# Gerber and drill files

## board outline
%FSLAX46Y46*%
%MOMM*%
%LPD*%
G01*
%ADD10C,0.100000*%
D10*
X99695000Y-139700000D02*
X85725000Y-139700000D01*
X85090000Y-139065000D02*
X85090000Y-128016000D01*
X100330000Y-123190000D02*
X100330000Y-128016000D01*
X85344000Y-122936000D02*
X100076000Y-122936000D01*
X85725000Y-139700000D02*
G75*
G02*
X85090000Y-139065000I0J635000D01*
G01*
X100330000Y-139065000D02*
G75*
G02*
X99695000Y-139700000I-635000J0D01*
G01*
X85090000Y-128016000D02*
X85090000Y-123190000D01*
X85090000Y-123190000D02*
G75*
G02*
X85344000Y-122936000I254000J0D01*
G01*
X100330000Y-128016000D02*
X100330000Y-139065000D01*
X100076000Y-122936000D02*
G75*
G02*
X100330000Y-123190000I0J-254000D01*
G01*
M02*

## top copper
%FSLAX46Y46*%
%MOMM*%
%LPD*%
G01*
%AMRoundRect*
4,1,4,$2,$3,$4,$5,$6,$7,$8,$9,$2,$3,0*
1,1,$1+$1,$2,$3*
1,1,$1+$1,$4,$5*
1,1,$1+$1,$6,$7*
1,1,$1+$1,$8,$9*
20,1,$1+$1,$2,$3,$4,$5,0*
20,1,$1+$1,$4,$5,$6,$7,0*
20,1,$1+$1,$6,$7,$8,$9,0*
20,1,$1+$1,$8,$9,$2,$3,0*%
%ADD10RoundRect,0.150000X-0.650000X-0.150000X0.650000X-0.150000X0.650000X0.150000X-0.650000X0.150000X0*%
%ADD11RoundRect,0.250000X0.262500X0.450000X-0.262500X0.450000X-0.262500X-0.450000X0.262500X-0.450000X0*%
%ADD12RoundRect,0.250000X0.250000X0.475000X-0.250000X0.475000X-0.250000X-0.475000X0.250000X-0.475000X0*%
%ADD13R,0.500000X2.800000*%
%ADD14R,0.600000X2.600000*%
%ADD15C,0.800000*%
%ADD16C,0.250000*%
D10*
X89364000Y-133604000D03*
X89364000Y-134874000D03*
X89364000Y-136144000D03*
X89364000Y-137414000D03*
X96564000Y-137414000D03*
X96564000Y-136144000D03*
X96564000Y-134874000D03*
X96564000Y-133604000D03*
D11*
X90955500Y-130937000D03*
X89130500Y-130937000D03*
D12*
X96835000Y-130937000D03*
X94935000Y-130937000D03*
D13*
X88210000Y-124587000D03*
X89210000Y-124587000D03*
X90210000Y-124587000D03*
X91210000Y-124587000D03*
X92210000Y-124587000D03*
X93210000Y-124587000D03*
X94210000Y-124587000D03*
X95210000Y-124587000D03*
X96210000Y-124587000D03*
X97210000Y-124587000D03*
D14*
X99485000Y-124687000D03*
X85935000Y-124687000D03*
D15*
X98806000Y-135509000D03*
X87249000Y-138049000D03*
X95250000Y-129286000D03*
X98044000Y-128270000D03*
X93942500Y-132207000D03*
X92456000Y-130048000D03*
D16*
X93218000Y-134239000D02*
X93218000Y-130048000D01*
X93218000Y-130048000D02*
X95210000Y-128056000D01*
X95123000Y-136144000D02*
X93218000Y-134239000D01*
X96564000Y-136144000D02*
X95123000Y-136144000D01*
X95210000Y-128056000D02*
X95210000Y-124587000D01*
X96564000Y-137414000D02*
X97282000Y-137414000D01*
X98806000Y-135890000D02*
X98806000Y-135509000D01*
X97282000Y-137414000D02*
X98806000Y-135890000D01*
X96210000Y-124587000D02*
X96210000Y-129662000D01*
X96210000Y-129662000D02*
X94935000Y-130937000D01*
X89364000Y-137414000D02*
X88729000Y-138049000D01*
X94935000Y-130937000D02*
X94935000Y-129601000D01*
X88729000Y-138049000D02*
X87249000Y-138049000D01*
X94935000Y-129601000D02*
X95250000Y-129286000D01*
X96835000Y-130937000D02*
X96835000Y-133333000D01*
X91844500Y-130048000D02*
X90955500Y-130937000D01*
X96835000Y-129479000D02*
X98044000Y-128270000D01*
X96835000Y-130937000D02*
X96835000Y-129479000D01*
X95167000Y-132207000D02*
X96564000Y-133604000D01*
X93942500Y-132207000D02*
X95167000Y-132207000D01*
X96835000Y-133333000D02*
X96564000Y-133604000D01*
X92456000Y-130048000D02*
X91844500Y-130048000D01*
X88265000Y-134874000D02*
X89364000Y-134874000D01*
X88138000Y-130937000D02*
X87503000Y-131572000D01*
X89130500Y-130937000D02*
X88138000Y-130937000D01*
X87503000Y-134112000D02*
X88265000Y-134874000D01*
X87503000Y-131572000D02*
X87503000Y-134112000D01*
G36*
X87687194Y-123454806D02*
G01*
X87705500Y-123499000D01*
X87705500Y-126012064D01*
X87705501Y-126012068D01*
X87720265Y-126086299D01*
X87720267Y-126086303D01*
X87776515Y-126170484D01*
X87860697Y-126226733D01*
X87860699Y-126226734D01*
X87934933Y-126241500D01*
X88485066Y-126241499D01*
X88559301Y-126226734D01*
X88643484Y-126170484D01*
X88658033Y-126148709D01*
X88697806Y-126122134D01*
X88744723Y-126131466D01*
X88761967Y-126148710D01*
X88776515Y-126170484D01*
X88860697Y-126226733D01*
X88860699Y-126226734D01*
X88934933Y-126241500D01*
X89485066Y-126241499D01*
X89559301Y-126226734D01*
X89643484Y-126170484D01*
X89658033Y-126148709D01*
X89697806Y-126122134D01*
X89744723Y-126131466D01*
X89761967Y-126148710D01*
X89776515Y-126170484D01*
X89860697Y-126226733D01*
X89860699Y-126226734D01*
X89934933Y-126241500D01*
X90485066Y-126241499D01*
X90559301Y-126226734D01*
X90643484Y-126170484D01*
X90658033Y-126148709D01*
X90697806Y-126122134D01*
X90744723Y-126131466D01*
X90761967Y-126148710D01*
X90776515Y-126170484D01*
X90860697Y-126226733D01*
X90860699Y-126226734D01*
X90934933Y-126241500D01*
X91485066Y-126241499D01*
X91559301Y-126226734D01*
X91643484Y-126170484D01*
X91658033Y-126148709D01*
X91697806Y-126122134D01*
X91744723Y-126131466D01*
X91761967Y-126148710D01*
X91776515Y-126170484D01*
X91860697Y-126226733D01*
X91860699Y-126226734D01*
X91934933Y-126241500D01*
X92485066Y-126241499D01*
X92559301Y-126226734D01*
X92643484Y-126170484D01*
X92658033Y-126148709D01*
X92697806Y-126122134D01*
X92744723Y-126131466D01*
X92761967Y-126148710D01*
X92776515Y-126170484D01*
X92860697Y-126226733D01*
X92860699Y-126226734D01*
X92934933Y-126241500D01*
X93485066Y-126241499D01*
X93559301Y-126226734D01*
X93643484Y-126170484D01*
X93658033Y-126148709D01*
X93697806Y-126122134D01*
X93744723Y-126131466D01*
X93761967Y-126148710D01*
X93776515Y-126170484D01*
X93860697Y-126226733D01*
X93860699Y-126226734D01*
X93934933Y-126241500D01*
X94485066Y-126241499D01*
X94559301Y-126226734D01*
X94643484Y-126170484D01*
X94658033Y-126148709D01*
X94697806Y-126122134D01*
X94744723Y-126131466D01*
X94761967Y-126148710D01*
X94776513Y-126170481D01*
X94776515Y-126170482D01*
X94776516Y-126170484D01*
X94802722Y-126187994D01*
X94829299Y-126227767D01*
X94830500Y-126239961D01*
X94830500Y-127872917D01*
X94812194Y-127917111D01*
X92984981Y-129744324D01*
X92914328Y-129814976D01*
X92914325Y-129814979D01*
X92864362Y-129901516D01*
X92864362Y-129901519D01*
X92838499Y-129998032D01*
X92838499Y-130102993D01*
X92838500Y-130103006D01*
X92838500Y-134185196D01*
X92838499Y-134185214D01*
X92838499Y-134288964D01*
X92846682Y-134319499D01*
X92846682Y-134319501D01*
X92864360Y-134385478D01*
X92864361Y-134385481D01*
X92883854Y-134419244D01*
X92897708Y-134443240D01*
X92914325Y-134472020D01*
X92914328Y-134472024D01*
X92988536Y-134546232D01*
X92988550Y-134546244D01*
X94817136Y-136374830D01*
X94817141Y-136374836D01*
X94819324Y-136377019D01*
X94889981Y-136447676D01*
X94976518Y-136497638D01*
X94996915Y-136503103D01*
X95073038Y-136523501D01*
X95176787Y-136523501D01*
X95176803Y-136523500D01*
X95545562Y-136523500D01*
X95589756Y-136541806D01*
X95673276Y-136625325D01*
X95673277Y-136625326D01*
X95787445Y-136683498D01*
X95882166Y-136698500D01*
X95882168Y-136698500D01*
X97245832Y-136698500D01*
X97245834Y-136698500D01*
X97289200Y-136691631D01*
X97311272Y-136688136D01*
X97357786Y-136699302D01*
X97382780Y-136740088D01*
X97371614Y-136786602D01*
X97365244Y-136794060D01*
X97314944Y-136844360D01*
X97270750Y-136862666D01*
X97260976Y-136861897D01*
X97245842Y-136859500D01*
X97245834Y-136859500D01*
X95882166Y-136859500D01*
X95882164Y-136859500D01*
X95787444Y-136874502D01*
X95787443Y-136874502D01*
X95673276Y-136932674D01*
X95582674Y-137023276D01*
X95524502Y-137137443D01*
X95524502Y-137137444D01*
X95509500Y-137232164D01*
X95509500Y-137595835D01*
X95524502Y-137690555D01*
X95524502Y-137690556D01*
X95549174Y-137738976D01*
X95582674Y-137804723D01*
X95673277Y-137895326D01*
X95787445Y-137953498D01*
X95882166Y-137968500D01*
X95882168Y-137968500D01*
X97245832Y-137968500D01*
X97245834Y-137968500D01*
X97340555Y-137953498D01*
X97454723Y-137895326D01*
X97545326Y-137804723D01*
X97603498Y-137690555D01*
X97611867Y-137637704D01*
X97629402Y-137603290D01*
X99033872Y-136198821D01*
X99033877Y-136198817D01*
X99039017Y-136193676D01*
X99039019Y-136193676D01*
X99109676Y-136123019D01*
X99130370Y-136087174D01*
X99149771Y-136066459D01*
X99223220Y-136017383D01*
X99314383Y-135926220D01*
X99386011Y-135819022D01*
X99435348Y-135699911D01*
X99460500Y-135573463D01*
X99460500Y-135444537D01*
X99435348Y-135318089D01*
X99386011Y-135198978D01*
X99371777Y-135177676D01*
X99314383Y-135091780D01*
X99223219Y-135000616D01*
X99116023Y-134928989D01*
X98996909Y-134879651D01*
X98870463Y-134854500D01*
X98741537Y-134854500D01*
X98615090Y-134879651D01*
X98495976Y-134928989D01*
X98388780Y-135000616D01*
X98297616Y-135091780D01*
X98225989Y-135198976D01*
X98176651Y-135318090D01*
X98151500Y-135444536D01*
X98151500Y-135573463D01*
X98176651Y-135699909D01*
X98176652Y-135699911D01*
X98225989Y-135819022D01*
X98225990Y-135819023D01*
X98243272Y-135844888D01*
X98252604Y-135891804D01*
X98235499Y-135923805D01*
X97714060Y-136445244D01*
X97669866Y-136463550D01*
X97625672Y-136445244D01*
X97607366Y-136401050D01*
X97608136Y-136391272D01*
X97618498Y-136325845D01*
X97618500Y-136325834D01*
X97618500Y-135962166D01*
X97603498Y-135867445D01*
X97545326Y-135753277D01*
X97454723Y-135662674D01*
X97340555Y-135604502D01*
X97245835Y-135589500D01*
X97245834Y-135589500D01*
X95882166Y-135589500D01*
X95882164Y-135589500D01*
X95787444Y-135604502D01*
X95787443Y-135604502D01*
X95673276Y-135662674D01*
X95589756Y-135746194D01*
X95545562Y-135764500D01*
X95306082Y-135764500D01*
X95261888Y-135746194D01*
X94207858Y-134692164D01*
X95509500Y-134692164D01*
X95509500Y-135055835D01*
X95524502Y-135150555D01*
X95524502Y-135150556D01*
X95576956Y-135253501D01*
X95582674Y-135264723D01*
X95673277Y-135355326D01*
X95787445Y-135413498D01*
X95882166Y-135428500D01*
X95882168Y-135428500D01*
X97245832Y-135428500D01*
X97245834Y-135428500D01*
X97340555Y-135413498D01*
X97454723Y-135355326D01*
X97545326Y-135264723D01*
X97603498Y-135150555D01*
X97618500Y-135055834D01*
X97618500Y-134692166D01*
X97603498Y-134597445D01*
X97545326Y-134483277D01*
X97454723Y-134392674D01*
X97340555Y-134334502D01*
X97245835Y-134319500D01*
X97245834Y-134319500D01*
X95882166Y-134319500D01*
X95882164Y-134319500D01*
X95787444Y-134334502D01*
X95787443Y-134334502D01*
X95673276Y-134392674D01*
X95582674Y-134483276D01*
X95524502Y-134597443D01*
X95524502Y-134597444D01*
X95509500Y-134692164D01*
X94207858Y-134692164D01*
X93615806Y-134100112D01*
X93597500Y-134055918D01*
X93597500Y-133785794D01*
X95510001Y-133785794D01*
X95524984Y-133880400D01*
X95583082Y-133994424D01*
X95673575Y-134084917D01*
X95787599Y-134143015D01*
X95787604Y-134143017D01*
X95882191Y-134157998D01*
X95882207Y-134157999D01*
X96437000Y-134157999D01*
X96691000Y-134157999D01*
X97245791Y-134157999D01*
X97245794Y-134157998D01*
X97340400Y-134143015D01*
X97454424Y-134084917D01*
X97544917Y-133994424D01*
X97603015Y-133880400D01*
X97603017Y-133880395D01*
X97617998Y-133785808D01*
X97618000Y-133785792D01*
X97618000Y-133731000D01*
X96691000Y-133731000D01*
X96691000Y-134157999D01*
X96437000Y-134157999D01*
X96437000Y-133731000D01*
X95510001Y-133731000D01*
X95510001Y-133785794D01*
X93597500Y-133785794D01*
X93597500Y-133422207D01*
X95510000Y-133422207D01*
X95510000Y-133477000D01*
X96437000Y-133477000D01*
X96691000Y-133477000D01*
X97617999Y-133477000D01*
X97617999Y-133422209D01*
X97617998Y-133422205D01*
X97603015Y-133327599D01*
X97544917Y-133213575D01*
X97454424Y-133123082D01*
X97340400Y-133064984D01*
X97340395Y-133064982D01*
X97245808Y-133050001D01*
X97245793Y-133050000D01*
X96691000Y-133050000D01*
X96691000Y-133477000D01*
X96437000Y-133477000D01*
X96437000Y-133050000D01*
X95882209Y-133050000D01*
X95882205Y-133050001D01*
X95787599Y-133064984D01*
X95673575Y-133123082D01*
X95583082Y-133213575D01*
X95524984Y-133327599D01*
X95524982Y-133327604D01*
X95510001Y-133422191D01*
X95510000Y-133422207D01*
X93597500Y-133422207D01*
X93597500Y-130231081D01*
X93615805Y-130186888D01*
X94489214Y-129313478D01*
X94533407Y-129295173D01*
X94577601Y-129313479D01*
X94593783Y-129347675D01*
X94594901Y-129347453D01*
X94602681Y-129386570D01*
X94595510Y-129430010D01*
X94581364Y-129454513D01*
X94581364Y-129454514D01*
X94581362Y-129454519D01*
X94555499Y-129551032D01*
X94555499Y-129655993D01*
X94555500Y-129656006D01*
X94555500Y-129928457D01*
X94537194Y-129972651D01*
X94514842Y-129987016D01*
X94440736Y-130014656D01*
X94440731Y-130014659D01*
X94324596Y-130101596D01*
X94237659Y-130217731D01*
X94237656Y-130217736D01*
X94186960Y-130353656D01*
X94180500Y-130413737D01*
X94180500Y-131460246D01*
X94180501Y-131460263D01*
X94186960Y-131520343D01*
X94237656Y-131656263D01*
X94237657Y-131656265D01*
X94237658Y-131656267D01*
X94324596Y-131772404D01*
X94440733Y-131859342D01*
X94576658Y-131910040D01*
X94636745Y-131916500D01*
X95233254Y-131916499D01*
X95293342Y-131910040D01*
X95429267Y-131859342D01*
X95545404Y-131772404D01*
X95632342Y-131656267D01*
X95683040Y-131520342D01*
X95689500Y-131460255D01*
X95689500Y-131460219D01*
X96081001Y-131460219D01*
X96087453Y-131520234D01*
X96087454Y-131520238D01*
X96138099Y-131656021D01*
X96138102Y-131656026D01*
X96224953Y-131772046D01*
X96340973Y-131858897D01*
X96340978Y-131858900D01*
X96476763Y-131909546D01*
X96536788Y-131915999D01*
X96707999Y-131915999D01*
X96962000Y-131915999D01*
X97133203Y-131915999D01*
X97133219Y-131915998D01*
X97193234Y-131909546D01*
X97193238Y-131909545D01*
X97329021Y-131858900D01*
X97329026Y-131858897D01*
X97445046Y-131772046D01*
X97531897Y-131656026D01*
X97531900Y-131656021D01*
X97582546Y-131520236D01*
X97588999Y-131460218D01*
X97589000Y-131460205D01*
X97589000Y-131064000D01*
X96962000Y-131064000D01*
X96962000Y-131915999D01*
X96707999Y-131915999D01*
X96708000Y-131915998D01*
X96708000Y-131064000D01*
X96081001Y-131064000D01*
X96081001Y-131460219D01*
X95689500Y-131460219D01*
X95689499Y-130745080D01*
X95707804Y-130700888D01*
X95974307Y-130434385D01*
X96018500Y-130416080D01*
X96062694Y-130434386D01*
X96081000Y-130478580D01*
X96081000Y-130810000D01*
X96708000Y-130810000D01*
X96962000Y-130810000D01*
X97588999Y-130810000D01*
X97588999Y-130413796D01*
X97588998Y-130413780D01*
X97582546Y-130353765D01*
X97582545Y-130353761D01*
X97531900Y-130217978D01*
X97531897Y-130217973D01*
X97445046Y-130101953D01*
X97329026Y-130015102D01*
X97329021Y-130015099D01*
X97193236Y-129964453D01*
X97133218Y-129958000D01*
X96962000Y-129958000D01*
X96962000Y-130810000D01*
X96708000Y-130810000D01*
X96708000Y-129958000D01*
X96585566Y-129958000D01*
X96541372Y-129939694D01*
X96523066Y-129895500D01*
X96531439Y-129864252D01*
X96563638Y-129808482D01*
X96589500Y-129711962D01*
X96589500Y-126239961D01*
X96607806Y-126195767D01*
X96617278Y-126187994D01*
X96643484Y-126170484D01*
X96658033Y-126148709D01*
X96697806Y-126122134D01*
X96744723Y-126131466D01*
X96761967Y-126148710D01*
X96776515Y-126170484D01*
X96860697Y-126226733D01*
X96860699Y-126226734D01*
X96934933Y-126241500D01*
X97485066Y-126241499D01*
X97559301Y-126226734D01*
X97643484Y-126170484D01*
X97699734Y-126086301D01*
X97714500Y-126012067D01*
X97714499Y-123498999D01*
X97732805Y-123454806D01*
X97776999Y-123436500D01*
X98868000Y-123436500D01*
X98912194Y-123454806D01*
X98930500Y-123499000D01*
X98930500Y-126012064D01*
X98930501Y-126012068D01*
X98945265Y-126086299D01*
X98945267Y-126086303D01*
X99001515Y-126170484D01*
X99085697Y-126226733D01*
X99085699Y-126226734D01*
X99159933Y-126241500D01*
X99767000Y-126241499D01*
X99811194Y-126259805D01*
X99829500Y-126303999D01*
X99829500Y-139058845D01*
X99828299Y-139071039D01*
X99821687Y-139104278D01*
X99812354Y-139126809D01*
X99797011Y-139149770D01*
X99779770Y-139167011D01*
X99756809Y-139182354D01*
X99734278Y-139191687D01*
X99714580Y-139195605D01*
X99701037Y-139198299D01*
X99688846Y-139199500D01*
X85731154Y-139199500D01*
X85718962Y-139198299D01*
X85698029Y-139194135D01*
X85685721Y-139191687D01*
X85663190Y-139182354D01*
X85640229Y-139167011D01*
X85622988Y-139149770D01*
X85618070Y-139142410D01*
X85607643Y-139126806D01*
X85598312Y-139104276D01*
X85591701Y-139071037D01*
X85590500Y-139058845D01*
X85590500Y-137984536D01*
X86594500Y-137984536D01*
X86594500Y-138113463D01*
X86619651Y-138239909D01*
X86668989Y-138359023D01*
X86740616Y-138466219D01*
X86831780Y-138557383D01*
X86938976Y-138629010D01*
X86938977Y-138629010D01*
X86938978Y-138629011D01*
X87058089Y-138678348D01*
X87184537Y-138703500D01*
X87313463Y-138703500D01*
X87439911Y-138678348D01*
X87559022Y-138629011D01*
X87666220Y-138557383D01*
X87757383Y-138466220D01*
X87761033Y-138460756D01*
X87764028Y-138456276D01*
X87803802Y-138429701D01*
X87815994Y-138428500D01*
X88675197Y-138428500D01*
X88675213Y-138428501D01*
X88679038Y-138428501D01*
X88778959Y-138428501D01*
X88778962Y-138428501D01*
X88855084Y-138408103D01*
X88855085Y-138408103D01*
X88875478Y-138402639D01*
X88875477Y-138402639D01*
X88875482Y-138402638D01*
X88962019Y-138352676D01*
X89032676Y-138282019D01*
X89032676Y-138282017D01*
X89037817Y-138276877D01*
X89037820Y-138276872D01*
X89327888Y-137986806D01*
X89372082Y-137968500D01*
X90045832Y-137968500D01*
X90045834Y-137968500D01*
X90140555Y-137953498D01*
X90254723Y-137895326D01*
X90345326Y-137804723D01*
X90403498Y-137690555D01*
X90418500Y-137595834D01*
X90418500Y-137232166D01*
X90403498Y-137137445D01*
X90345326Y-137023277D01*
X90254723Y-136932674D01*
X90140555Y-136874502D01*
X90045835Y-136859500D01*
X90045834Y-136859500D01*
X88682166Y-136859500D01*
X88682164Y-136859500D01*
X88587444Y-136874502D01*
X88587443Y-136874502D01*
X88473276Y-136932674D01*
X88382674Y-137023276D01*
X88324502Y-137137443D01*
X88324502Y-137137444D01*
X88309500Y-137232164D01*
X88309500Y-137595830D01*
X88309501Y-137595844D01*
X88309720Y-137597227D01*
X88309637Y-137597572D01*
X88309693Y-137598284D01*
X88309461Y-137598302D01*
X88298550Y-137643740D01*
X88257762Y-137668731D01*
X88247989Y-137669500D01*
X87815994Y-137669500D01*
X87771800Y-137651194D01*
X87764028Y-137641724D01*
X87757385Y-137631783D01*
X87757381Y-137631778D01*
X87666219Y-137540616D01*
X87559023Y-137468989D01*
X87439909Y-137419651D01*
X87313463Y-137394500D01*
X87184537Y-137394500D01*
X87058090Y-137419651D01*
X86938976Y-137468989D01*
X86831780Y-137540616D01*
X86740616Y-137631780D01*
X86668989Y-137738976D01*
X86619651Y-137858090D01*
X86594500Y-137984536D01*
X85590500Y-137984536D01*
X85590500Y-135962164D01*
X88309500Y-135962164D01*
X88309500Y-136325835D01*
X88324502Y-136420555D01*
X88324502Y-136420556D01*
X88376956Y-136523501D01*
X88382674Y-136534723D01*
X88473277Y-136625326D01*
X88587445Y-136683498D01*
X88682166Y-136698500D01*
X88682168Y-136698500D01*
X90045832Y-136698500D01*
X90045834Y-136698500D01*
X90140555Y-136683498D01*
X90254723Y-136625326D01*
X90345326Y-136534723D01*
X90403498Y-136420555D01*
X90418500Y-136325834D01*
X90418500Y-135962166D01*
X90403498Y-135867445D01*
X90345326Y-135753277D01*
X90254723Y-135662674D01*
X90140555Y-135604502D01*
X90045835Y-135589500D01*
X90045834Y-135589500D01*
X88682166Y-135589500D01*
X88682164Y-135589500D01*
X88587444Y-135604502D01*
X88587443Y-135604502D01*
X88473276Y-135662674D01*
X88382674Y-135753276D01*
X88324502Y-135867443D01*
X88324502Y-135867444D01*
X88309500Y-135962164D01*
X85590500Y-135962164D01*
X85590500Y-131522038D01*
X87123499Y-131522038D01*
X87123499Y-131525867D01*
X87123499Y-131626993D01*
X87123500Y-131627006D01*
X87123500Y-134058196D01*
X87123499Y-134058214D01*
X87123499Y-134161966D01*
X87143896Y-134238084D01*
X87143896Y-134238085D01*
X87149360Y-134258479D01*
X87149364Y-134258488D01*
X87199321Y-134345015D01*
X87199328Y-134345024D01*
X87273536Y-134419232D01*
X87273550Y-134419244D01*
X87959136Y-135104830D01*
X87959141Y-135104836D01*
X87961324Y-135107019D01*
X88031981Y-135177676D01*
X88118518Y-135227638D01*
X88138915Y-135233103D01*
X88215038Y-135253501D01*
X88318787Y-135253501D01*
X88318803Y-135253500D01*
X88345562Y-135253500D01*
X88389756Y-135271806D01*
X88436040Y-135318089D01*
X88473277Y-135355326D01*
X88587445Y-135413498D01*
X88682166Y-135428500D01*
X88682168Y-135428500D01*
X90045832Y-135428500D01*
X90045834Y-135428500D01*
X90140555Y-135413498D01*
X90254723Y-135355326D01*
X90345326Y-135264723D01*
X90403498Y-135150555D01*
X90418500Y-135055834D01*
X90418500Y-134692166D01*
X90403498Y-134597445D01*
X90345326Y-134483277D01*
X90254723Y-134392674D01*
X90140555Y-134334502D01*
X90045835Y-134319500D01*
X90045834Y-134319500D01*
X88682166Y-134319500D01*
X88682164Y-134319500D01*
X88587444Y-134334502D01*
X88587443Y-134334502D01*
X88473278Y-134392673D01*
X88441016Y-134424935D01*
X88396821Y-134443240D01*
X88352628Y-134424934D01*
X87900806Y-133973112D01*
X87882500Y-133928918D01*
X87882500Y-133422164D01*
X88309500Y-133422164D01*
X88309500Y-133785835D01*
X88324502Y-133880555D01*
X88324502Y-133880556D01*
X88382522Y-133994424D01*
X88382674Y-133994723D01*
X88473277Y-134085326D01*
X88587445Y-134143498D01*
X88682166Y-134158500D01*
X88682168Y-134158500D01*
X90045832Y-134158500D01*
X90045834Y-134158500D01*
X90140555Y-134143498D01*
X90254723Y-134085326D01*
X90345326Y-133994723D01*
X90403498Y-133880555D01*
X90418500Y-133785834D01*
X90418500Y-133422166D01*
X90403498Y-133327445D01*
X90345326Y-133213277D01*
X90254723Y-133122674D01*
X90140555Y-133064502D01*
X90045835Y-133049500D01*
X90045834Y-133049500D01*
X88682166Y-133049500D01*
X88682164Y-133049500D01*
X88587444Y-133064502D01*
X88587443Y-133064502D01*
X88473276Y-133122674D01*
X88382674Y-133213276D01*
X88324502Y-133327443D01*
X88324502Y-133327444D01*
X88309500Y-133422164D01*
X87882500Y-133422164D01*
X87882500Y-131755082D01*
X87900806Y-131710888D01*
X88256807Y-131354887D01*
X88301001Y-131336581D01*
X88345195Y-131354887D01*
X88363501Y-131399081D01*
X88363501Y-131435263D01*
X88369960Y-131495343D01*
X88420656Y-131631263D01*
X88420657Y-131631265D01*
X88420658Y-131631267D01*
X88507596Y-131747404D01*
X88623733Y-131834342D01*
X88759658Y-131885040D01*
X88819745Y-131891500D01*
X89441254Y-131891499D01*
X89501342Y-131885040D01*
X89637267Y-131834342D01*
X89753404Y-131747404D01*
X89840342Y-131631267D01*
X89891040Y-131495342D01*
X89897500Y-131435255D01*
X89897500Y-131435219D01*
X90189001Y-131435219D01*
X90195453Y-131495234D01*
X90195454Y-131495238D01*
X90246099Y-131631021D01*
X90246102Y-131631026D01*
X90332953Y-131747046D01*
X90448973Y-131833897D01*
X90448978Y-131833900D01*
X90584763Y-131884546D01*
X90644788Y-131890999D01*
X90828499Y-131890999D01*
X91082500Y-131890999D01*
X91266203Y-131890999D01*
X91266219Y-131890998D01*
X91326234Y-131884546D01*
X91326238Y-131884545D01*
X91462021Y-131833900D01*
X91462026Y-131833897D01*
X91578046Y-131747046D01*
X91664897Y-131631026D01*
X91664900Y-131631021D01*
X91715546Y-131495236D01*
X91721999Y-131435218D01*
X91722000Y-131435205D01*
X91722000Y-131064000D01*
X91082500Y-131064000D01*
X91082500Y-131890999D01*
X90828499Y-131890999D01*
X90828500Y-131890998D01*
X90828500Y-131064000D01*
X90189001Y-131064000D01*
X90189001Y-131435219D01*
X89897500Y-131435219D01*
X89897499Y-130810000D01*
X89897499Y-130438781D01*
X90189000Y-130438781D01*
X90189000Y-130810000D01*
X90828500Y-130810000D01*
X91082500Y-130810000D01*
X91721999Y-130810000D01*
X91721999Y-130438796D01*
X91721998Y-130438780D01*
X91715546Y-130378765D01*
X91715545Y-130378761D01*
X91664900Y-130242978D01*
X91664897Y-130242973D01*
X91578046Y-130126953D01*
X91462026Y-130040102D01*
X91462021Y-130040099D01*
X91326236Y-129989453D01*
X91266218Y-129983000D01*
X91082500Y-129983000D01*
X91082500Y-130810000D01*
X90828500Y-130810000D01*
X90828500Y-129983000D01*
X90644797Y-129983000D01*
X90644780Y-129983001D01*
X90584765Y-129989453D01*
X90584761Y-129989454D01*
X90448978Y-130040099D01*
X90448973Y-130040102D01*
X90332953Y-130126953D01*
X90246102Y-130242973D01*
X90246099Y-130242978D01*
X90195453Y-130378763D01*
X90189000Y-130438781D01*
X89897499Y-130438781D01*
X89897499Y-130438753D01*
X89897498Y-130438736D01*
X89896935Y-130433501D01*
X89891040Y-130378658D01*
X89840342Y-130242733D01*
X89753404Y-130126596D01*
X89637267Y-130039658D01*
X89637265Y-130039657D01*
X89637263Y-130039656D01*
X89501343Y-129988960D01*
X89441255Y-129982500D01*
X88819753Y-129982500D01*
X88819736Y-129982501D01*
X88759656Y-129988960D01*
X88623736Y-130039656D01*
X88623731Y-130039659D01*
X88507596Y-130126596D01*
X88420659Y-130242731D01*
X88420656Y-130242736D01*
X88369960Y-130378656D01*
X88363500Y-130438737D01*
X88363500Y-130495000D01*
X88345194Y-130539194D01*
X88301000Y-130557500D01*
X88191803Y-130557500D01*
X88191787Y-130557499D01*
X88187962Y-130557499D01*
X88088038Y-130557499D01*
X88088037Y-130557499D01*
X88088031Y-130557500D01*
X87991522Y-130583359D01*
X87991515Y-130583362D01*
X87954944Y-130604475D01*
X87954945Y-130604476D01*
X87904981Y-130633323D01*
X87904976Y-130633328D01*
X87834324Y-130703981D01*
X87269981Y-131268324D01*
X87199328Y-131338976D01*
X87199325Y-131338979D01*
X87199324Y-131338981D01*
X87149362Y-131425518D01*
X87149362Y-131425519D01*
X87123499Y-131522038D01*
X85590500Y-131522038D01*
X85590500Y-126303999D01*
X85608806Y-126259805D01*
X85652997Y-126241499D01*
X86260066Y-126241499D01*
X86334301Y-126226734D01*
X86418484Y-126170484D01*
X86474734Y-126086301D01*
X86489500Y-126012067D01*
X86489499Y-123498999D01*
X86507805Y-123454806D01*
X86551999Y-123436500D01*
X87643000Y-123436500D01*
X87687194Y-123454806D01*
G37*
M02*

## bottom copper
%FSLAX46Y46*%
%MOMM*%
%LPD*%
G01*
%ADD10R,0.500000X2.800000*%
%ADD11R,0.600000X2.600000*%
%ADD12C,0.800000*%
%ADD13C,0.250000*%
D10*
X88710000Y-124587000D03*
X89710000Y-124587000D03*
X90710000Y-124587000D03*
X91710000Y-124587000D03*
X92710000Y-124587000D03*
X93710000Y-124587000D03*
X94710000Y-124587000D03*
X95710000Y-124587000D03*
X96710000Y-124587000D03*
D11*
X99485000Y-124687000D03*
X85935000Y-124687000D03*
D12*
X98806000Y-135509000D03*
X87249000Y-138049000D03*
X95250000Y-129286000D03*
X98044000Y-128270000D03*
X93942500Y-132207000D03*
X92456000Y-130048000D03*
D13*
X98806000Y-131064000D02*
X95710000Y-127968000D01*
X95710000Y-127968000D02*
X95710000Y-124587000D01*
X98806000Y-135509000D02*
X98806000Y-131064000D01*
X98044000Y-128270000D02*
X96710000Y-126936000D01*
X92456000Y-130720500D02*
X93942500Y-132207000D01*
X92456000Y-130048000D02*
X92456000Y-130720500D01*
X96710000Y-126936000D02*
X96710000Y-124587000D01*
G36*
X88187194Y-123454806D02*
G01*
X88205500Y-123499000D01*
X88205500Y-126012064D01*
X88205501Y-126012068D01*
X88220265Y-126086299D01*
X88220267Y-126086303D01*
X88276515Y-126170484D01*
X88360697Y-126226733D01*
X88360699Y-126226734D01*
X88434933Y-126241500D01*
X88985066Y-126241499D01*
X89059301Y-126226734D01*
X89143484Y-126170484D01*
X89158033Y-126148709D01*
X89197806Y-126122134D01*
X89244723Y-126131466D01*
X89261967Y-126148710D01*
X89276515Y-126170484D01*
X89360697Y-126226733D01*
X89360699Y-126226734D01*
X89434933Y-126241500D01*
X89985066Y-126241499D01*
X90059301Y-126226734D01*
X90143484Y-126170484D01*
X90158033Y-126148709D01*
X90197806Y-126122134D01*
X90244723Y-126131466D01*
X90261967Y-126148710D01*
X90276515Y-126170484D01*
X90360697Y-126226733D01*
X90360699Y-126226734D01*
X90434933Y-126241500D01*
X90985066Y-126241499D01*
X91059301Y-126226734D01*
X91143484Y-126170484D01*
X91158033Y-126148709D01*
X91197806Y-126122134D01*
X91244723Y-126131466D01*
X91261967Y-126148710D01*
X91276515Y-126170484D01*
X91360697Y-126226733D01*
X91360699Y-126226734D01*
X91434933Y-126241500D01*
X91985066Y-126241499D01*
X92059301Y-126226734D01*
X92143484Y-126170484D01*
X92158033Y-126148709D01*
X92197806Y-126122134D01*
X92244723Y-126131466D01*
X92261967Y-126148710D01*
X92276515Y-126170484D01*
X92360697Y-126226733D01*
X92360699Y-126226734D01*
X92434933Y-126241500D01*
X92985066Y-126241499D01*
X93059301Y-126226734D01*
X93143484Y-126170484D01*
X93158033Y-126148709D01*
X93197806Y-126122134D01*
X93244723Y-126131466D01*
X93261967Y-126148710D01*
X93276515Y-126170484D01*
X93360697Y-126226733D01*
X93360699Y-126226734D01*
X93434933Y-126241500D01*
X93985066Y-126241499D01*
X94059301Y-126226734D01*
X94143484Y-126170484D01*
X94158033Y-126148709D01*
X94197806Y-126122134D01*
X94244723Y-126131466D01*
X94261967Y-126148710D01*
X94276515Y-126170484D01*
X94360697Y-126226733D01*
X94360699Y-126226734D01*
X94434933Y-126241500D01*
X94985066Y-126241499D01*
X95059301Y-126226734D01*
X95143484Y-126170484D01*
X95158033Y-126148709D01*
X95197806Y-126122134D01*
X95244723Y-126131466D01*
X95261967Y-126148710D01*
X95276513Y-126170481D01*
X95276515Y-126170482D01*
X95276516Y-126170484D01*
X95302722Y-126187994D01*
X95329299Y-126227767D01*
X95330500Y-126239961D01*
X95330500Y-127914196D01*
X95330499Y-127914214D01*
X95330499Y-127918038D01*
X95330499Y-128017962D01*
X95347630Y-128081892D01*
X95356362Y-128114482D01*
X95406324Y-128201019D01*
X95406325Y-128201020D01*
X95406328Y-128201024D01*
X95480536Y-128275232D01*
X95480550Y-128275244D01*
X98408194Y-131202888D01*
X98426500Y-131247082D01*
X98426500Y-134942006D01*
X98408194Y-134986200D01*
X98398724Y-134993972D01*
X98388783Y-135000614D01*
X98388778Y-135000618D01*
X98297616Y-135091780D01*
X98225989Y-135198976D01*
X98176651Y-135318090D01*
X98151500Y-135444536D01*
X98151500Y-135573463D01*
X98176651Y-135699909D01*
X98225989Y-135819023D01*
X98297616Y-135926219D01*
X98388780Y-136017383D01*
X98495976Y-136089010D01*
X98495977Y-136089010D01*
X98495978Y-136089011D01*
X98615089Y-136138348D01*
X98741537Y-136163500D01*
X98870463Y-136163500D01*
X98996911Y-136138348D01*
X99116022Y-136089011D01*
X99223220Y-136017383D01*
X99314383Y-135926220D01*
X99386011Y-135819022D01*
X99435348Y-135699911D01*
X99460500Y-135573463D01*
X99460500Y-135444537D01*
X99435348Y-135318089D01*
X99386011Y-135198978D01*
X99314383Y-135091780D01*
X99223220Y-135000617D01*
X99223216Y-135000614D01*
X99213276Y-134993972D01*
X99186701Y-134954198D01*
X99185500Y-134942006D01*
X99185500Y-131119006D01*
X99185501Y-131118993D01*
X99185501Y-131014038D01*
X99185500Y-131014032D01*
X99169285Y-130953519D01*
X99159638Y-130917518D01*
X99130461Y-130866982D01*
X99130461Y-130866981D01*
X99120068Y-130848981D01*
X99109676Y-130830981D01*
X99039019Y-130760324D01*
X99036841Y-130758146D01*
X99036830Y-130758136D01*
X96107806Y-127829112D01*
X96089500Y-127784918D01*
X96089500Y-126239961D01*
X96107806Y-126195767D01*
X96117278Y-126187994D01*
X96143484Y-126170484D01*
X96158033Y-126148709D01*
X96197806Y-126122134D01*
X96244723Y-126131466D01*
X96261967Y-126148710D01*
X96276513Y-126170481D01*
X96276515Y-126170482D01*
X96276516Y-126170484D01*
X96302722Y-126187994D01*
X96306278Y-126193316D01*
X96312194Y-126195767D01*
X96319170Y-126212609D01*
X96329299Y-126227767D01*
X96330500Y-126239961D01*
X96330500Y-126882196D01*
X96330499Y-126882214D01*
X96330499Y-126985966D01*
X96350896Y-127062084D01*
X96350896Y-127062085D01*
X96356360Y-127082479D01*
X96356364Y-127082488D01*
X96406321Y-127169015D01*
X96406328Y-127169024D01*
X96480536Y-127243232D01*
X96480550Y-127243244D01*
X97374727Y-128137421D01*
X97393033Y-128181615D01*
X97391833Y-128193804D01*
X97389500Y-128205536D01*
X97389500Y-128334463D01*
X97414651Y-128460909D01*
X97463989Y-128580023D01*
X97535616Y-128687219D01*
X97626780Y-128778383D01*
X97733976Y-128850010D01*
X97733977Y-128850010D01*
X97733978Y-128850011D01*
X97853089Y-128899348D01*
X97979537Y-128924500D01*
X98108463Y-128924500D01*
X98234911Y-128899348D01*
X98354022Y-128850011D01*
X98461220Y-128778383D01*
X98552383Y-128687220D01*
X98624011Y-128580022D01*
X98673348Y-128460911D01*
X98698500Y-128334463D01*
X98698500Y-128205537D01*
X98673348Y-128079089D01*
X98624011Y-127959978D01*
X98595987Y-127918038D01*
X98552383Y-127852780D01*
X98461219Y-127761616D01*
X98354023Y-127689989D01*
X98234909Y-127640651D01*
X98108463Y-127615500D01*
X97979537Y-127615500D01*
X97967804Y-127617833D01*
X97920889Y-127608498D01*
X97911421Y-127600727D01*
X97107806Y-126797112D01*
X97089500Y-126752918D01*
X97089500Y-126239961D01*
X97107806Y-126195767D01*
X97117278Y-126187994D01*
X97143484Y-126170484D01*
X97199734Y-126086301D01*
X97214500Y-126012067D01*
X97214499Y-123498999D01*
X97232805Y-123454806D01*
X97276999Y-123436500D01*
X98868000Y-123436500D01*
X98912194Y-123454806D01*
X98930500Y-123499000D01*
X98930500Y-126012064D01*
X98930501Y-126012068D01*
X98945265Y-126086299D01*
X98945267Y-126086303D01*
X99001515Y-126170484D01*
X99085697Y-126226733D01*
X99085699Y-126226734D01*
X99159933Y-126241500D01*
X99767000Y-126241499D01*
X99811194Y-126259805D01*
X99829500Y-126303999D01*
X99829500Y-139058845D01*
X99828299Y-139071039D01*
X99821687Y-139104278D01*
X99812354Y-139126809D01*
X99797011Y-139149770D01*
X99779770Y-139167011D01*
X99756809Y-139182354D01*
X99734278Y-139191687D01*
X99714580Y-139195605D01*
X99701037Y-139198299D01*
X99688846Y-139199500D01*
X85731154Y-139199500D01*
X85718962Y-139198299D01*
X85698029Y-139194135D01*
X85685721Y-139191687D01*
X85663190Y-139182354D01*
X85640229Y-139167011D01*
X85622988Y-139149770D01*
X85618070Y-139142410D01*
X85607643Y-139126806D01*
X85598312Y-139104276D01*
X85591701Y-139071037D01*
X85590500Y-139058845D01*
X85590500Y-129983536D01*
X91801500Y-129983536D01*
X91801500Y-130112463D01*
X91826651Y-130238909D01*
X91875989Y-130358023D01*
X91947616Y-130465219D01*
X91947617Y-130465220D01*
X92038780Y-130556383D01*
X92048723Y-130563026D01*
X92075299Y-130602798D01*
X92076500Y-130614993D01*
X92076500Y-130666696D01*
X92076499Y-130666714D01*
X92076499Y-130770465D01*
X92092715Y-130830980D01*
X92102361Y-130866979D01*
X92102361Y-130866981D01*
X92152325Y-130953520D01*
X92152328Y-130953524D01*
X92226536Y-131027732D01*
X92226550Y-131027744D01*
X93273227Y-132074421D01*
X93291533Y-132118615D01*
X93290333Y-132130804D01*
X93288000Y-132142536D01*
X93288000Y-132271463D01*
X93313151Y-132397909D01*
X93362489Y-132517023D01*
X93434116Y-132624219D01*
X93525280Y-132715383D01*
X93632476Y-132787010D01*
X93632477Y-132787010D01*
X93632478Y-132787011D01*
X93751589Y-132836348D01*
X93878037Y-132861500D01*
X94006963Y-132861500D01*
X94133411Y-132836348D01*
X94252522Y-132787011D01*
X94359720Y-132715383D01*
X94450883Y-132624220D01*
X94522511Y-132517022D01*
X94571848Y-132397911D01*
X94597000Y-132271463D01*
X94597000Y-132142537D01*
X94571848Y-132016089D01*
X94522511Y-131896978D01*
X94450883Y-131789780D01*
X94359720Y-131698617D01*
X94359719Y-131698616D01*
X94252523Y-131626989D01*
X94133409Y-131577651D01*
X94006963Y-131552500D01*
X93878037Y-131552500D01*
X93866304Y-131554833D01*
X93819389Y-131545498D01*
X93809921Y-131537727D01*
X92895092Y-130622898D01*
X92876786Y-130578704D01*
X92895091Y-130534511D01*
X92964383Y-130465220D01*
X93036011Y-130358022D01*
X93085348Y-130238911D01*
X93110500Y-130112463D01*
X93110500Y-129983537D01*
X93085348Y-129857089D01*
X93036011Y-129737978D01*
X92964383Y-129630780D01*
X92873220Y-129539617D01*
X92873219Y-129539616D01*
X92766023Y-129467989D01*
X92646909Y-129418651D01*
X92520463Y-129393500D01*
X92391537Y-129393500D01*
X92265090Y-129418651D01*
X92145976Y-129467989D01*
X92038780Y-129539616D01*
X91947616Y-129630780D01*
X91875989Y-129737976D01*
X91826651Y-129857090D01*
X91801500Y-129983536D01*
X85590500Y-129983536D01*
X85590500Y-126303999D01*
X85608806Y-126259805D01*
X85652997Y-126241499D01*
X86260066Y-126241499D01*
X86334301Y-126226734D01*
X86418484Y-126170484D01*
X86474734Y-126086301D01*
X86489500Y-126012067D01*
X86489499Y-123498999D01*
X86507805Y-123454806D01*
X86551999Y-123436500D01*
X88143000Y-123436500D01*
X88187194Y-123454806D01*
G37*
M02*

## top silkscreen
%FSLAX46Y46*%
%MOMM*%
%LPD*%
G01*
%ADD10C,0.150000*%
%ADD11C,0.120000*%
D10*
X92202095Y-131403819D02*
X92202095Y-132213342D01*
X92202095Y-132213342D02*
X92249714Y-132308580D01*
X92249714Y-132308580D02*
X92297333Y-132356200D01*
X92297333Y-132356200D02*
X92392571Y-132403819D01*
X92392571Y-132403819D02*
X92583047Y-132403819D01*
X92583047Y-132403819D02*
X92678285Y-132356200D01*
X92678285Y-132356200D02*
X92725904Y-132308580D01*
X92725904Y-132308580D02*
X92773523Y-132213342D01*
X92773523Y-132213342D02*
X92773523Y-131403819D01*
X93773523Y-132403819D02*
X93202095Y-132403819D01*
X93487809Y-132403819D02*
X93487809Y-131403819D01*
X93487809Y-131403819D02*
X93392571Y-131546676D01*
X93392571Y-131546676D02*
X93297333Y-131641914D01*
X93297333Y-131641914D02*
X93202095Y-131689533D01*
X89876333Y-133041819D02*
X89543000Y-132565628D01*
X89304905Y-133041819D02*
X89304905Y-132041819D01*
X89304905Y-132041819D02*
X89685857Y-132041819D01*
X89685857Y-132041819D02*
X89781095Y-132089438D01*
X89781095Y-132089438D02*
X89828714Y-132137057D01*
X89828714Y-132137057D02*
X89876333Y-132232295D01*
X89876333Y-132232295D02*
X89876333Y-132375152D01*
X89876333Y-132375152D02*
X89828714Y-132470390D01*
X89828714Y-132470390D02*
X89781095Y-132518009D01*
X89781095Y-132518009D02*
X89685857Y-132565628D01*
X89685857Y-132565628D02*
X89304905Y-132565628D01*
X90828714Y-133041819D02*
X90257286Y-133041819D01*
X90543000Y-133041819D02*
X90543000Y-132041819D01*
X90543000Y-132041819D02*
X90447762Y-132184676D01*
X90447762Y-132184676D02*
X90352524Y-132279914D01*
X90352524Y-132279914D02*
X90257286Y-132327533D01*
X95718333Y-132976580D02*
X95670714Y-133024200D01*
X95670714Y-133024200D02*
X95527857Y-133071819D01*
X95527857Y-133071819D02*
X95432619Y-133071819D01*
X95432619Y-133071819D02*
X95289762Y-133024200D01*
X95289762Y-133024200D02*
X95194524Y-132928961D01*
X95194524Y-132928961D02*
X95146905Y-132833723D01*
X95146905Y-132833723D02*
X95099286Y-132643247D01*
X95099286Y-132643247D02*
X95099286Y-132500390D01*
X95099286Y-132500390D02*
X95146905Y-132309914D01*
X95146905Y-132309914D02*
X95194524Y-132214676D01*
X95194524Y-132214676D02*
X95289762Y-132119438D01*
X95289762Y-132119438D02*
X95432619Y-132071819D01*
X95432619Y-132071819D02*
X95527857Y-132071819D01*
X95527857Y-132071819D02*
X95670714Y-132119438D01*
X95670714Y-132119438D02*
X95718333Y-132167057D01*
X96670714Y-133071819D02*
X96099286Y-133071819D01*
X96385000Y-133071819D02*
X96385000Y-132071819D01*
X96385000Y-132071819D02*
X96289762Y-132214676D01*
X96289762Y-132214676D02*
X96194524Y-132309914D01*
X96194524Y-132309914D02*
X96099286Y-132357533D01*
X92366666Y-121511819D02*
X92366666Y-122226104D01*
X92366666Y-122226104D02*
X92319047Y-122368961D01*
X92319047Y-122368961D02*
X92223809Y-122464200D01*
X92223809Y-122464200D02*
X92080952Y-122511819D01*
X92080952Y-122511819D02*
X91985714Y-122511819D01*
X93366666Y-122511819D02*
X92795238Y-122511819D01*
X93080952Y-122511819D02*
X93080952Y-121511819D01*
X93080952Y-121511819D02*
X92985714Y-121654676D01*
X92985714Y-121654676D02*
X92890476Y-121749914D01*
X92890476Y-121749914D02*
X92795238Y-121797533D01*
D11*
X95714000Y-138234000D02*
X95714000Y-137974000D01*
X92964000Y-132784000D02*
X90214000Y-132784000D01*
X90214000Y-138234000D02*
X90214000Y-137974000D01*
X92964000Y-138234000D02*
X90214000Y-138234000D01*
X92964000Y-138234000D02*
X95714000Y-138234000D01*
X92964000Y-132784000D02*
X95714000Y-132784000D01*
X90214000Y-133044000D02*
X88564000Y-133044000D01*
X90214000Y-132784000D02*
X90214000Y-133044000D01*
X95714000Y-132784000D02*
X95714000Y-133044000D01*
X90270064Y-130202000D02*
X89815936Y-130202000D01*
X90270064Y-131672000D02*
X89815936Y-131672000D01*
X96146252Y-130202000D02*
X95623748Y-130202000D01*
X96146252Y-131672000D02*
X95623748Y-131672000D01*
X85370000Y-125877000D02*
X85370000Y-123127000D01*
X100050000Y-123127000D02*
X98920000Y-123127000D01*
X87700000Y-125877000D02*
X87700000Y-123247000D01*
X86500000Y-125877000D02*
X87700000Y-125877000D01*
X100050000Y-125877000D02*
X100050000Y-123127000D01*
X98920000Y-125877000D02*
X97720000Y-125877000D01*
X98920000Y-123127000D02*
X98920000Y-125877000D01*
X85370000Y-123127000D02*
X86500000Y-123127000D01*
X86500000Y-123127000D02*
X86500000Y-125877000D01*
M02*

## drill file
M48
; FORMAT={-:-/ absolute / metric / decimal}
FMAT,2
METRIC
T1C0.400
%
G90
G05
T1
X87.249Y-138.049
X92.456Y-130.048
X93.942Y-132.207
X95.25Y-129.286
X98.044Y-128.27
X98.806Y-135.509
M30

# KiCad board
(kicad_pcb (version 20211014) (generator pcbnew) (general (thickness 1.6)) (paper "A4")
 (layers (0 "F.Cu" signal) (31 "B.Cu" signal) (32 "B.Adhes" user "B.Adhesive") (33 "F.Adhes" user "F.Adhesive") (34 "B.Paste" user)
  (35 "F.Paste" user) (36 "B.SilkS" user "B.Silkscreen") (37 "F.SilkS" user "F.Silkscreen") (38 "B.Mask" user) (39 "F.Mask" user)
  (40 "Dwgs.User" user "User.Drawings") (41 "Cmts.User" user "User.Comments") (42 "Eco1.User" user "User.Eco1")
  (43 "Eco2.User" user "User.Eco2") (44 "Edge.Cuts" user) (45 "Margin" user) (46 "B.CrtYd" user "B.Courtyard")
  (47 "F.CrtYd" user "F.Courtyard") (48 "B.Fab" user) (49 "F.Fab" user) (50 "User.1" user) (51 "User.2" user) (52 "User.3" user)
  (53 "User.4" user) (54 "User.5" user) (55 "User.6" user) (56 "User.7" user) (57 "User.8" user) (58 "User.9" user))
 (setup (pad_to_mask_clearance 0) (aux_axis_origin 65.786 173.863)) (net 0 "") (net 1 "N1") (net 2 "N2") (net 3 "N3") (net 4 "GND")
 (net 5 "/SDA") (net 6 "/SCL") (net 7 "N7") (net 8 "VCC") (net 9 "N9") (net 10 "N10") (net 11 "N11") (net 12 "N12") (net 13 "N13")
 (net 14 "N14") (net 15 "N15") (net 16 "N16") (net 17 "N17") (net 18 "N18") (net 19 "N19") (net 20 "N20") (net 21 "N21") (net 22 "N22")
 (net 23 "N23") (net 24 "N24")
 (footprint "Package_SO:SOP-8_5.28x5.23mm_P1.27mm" (layer "F.Cu") (at 92.964 135.509) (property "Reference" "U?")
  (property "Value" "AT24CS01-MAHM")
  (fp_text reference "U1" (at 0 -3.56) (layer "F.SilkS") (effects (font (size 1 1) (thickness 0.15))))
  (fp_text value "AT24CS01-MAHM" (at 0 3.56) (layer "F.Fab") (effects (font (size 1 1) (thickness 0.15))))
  (fp_line (start 2.75 2.725) (end 2.75 2.465) (layer "F.SilkS") (width 0.12))
  (fp_line (start 0 -2.725) (end -2.75 -2.725) (layer "F.SilkS") (width 0.12))
  (fp_line (start -2.75 2.725) (end -2.75 2.465) (layer "F.SilkS") (width 0.12))
  (fp_line (start 0 2.725) (end -2.75 2.725) (layer "F.SilkS") (width 0.12))
  (fp_line (start 0 2.725) (end 2.75 2.725) (layer "F.SilkS") (width 0.12))
  (fp_line (start 0 -2.725) (end 2.75 -2.725) (layer "F.SilkS") (width 0.12))
  (fp_line (start -2.75 -2.465) (end -4.4 -2.465) (layer "F.SilkS") (width 0.12))
  (fp_line (start -2.75 -2.725) (end -2.75 -2.465) (layer "F.SilkS") (width 0.12))
  (fp_line (start 2.75 -2.725) (end 2.75 -2.465) (layer "F.SilkS") (width 0.12))
  (pad "1" smd roundrect (at -3.6 -1.905) (size 1.6 0.6) (layers "F.Cu" "F.Paste" "F.Mask") (roundrect_rratio 0.25) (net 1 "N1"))
  (pad "2" smd roundrect (at -3.6 -0.635) (size 1.6 0.6) (layers "F.Cu" "F.Paste" "F.Mask") (roundrect_rratio 0.25) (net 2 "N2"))
  (pad "3" smd roundrect (at -3.6 0.635) (size 1.6 0.6) (layers "F.Cu" "F.Paste" "F.Mask") (roundrect_rratio 0.25) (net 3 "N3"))
  (pad "4" smd roundrect (at -3.6 1.905) (size 1.6 0.6) (layers "F.Cu" "F.Paste" "F.Mask") (roundrect_rratio 0.25) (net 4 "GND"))
  (pad "5" smd roundrect (at 3.6 1.905) (size 1.6 0.6) (layers "F.Cu" "F.Paste" "F.Mask") (roundrect_rratio 0.25) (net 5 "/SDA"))
  (pad "6" smd roundrect (at 3.6 0.635) (size 1.6 0.6) (layers "F.Cu" "F.Paste" "F.Mask") (roundrect_rratio 0.25) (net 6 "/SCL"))
  (pad "7" smd roundrect (at 3.6 -0.635) (size 1.6 0.6) (layers "F.Cu" "F.Paste" "F.Mask") (roundrect_rratio 0.25) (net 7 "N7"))
  (pad "8" smd roundrect (at 3.6 -1.905) (size 1.6 0.6) (layers "F.Cu" "F.Paste" "F.Mask") (roundrect_rratio 0.25) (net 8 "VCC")))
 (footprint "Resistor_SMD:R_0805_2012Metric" (layer "F.Cu") (at 90.043 130.937 180) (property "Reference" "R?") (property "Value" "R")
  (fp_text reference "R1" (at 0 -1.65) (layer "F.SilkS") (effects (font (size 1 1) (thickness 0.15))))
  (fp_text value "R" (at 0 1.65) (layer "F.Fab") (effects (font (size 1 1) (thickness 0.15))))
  (fp_line (start -0.227064 0.735) (end 0.227064 0.735) (layer "F.SilkS") (width 0.12))
  (fp_line (start -0.227064 -0.735) (end 0.227064 -0.735) (layer "F.SilkS") (width 0.12))
  (pad "1" smd roundrect (at -0.9125 0 180) (size 1.025 1.4) (layers "F.Cu" "F.Paste" "F.Mask") (roundrect_rratio 0.243902) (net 8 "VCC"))
  (pad "2" smd roundrect (at 0.9125 0 180) (size 1.025 1.4) (layers "F.Cu" "F.Paste" "F.Mask") (roundrect_rratio 0.243902) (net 2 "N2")))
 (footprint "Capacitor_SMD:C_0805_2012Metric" (layer "F.Cu") (at 95.885 130.937 180) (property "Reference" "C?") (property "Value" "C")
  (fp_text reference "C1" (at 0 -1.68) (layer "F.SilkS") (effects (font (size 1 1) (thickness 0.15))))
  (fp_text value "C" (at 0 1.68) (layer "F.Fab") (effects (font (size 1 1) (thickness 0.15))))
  (fp_line (start -0.261252 0.735) (end 0.261252 0.735) (layer "F.SilkS") (width 0.12))
  (fp_line (start -0.261252 -0.735) (end 0.261252 -0.735) (layer "F.SilkS") (width 0.12))
  (pad "1" smd roundrect (at -0.95 0 180) (size 1 1.45) (layers "F.Cu" "F.Paste" "F.Mask") (roundrect_rratio 0.25) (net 8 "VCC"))
  (pad "2" smd roundrect (at 0.95 0 180) (size 1 1.45) (layers "F.Cu" "F.Paste" "F.Mask") (roundrect_rratio 0.25) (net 4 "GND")))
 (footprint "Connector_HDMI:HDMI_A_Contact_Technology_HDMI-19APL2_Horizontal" (layer "F.Cu") (at 92.71 124.587)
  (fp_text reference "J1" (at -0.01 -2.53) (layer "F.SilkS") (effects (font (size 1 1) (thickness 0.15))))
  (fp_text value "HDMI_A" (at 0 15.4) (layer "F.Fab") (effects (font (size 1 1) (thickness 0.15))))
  (fp_line (start -7.34 1.29) (end -7.34 -1.46) (layer "F.SilkS") (width 0.12))
  (fp_line (start 7.34 -1.46) (end 6.21 -1.46) (layer "F.SilkS") (width 0.12))
  (fp_line (start -5.01 1.29) (end -5.01 -1.34) (layer "F.SilkS") (width 0.12))
  (fp_line (start -6.21 1.29) (end -5.01 1.29) (layer "F.SilkS") (width 0.12))
  (fp_line (start 7.34 1.29) (end 7.34 -1.46) (layer "F.SilkS") (width 0.12))
  (fp_line (start 6.21 1.29) (end 5.01 1.29) (layer "F.SilkS") (width 0.12))
  (fp_line (start 6.21 -1.46) (end 6.21 1.29) (layer "F.SilkS") (width 0.12))
  (fp_line (start -7.34 -1.46) (end -6.21 -1.46) (layer "F.SilkS") (width 0.12))
  (fp_line (start -6.21 -1.46) (end -6.21 1.29) (layer "F.SilkS") (width 0.12))
  (pad "1" smd rect (at -4.5 0) (size 0.5 2.8) (layers "F.Cu" "F.Paste" "F.Mask") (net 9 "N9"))
  (pad "2" smd rect (at -4 0) (size 0.5 2.8) (layers "B.Cu" "B.Paste" "B.Mask") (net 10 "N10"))
  (pad "3" smd rect (at -3.5 0) (size 0.5 2.8) (layers "F.Cu" "F.Paste" "F.Mask") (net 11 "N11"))
  (pad "4" smd rect (at -3 0) (size 0.5 2.8) (layers "B.Cu" "B.Paste" "B.Mask") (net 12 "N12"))
  (pad "5" smd rect (at -2.5 0) (size 0.5 2.8) (layers "F.Cu" "F.Paste" "F.Mask") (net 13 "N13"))
  (pad "6" smd rect (at -2 0) (size 0.5 2.8) (layers "B.Cu" "B.Paste" "B.Mask") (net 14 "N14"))
  (pad "7" smd rect (at -1.5 0) (size 0.5 2.8) (layers "F.Cu" "F.Paste" "F.Mask") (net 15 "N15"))
  (pad "8" smd rect (at -1 0) (size 0.5 2.8) (layers "B.Cu" "B.Paste" "B.Mask") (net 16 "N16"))
  (pad "9" smd rect (at -0.5 0) (size 0.5 2.8) (layers "F.Cu" "F.Paste" "F.Mask") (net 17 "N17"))
  (pad "10" smd rect (at 0 0) (size 0.5 2.8) (layers "B.Cu" "B.Paste" "B.Mask") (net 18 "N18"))
  (pad "11" smd rect (at 0.5 0) (size 0.5 2.8) (layers "F.Cu" "F.Paste" "F.Mask") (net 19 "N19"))
  (pad "12" smd rect (at 1 0) (size 0.5 2.8) (layers "B.Cu" "B.Paste" "B.Mask") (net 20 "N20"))
  (pad "13" smd rect (at 1.5 0) (size 0.5 2.8) (layers "F.Cu" "F.Paste" "F.Mask") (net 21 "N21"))
  (pad "14" smd rect (at 2 0) (size 0.5 2.8) (layers "B.Cu" "B.Paste" "B.Mask") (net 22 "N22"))
  (pad "15" smd rect (at 2.5 0) (size 0.5 2.8) (layers "F.Cu" "F.Paste" "F.Mask") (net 6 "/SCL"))
  (pad "16" smd rect (at 3 0) (size 0.5 2.8) (layers "B.Cu" "B.Paste" "B.Mask") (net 5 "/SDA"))
  (pad "17" smd rect (at 3.5 0) (size 0.5 2.8) (layers "F.Cu" "F.Paste" "F.Mask") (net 4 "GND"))
  (pad "18" smd rect (at 4 0) (size 0.5 2.8) (layers "B.Cu" "B.Paste" "B.Mask") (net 8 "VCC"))
  (pad "19" smd rect (at 4.5 0) (size 0.5 2.8) (layers "F.Cu" "F.Paste" "F.Mask") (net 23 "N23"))
  (pad "SH" smd rect (at 6.775 0.1) (size 0.6 2.6) (layers "F.Cu" "F.Paste" "F.Mask") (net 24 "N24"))
  (pad "SH" smd rect (at -6.775 0.1) (size 0.6 2.6) (layers "F.Cu" "F.Paste" "F.Mask") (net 24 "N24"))
  (pad "SH" smd rect (at 6.775 0.1) (size 0.6 2.6) (layers "B.Cu" "B.Paste" "B.Mask") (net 24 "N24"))
  (pad "SH" smd rect (at -6.775 0.1) (size 0.6 2.6) (layers "B.Cu" "B.Paste" "B.Mask") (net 24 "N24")))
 (gr_line (start 99.695 139.7) (end 85.725 139.7) (layer "Edge.Cuts") (width 0.1))
 (gr_line (start 85.09 139.065) (end 85.09 128.016) (layer "Edge.Cuts") (width 0.1))
 (gr_line (start 100.33 123.19) (end 100.33 128.016) (layer "Edge.Cuts") (width 0.1))
 (gr_line (start 85.344 122.936) (end 100.076 122.936) (layer "Edge.Cuts") (width 0.1))
 (gr_arc (start 85.725 139.7) (mid 85.275987 139.514013) (end 85.09 139.065) (layer "Edge.Cuts") (width 0.1))
 (gr_arc (start 100.33 139.065) (mid 100.144013 139.514013) (end 99.695 139.7) (layer "Edge.Cuts") (width 0.1))
 (gr_line (start 85.09 128.016) (end 85.09 123.19) (layer "Edge.Cuts") (width 0.1))
 (gr_arc (start 85.09 123.19) (mid 85.164395 123.010395) (end 85.344 122.936) (layer "Edge.Cuts") (width 0.1))
 (gr_line (start 100.33 128.016) (end 100.33 139.065) (layer "Edge.Cuts") (width 0.1))
 (gr_arc (start 100.076 122.936) (mid 100.255605 123.010395) (end 100.33 123.19) (layer "Edge.Cuts") (width 0.1))
 (segment (start 93.218 134.239) (end 93.218 130.048) (width 0.25) (layer "F.Cu") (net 6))
 (segment (start 93.218 130.048) (end 95.21 128.056) (width 0.25) (layer "F.Cu") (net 6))
 (segment (start 95.123 136.144) (end 93.218 134.239) (width 0.25) (layer "F.Cu") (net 6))
 (segment (start 96.564 136.144) (end 95.123 136.144) (width 0.25) (layer "F.Cu") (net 6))
 (segment (start 95.21 128.056) (end 95.21 124.587) (width 0.25) (layer "F.Cu") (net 6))
 (segment (start 96.564 137.414) (end 97.282 137.414) (width 0.25) (layer "F.Cu") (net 5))
 (segment (start 98.806 135.89) (end 98.806 135.509) (width 0.25) (layer "F.Cu") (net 5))
 (segment (start 97.282 137.414) (end 98.806 135.89) (width 0.25) (layer "F.Cu") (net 5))
 (via (at 98.806 135.509) (size 0.8) (drill 0.4) (layers "F.Cu" "B.Cu") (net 5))
 (segment (start 98.806 131.064) (end 95.71 127.968) (width 0.25) (layer "B.Cu") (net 5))
 (segment (start 95.71 127.968) (end 95.71 124.587) (width 0.25) (layer "B.Cu") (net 5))
 (segment (start 98.806 135.509) (end 98.806 131.064) (width 0.25) (layer "B.Cu") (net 5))
 (segment (start 96.21 124.587) (end 96.21 129.662) (width 0.25) (layer "F.Cu") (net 4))
 (segment (start 96.21 129.662) (end 94.935 130.937) (width 0.25) (layer "F.Cu") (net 4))
 (segment (start 89.364 137.414) (end 88.729 138.049) (width 0.25) (layer "F.Cu") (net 4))
 (segment (start 94.935 130.937) (end 94.935 129.601) (width 0.25) (layer "F.Cu") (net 4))
 (segment (start 88.729 138.049) (end 87.249 138.049) (width 0.25) (layer "F.Cu") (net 4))
 (segment (start 94.935 129.601) (end 95.25 129.286) (width 0.25) (layer "F.Cu") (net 4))
 (via (at 87.249 138.049) (size 0.8) (drill 0.4) (layers "F.Cu" "B.Cu") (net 4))
 (via (at 95.25 129.286) (size 0.8) (drill 0.4) (layers "F.Cu" "B.Cu") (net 4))
 (segment (start 96.835 130.937) (end 96.835 133.333) (width 0.25) (layer "F.Cu") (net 8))
 (segment (start 91.8445 130.048) (end 90.9555 130.937) (width 0.25) (layer "F.Cu") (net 8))
 (segment (start 96.835 129.479) (end 98.044 128.27) (width 0.25) (layer "F.Cu") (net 8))
 (segment (start 96.835 130.937) (end 96.835 129.479) (width 0.25) (layer "F.Cu") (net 8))
 (segment (start 95.167 132.207) (end 96.564 133.604) (width 0.25) (layer "F.Cu") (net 8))
 (segment (start 93.9425 132.207) (end 95.167 132.207) (width 0.25) (layer "F.Cu") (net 8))
 (segment (start 96.835 133.333) (end 96.564 133.604) (width 0.25) (layer "F.Cu") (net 8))
 (segment (start 92.456 130.048) (end 91.8445 130.048) (width 0.25) (layer "F.Cu") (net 8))
 (via (at 98.044 128.27) (size 0.8) (drill 0.4) (layers "F.Cu" "B.Cu") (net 8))
 (via (at 93.9425 132.207) (size 0.8) (drill 0.4) (layers "F.Cu" "B.Cu") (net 8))
 (via (at 92.456 130.048) (size 0.8) (drill 0.4) (layers "F.Cu" "B.Cu") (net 8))
 (segment (start 98.044 128.27) (end 96.71 126.936) (width 0.25) (layer "B.Cu") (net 8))
 (segment (start 92.456 130.7205) (end 93.9425 132.207) (width 0.25) (layer "B.Cu") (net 8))
 (segment (start 92.456 130.048) (end 92.456 130.7205) (width 0.25) (layer "B.Cu") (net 8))
 (segment (start 96.71 126.936) (end 96.71 124.587) (width 0.25) (layer "B.Cu") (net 8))
 (segment (start 88.265 134.874) (end 89.364 134.874) (width 0.25) (layer "F.Cu") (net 2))
 (segment (start 88.138 130.937) (end 87.503 131.572) (width 0.25) (layer "F.Cu") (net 2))
 (segment (start 89.1305 130.937) (end 88.138 130.937) (width 0.25) (layer "F.Cu") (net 2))
 (segment (start 87.503 134.112) (end 88.265 134.874) (width 0.25) (layer "F.Cu") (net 2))
 (segment (start 87.503 131.572) (end 87.503 134.112) (width 0.25) (layer "F.Cu") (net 2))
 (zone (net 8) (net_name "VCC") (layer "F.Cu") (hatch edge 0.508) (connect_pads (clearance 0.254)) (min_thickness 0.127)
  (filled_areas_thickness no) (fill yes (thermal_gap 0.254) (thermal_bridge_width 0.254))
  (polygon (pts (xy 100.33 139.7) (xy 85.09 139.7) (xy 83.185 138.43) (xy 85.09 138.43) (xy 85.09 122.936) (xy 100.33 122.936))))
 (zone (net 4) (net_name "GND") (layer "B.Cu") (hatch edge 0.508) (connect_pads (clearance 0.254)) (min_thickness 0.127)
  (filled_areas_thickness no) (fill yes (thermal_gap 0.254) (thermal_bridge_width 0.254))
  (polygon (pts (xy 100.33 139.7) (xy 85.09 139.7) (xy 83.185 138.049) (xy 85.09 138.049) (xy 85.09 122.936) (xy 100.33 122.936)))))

